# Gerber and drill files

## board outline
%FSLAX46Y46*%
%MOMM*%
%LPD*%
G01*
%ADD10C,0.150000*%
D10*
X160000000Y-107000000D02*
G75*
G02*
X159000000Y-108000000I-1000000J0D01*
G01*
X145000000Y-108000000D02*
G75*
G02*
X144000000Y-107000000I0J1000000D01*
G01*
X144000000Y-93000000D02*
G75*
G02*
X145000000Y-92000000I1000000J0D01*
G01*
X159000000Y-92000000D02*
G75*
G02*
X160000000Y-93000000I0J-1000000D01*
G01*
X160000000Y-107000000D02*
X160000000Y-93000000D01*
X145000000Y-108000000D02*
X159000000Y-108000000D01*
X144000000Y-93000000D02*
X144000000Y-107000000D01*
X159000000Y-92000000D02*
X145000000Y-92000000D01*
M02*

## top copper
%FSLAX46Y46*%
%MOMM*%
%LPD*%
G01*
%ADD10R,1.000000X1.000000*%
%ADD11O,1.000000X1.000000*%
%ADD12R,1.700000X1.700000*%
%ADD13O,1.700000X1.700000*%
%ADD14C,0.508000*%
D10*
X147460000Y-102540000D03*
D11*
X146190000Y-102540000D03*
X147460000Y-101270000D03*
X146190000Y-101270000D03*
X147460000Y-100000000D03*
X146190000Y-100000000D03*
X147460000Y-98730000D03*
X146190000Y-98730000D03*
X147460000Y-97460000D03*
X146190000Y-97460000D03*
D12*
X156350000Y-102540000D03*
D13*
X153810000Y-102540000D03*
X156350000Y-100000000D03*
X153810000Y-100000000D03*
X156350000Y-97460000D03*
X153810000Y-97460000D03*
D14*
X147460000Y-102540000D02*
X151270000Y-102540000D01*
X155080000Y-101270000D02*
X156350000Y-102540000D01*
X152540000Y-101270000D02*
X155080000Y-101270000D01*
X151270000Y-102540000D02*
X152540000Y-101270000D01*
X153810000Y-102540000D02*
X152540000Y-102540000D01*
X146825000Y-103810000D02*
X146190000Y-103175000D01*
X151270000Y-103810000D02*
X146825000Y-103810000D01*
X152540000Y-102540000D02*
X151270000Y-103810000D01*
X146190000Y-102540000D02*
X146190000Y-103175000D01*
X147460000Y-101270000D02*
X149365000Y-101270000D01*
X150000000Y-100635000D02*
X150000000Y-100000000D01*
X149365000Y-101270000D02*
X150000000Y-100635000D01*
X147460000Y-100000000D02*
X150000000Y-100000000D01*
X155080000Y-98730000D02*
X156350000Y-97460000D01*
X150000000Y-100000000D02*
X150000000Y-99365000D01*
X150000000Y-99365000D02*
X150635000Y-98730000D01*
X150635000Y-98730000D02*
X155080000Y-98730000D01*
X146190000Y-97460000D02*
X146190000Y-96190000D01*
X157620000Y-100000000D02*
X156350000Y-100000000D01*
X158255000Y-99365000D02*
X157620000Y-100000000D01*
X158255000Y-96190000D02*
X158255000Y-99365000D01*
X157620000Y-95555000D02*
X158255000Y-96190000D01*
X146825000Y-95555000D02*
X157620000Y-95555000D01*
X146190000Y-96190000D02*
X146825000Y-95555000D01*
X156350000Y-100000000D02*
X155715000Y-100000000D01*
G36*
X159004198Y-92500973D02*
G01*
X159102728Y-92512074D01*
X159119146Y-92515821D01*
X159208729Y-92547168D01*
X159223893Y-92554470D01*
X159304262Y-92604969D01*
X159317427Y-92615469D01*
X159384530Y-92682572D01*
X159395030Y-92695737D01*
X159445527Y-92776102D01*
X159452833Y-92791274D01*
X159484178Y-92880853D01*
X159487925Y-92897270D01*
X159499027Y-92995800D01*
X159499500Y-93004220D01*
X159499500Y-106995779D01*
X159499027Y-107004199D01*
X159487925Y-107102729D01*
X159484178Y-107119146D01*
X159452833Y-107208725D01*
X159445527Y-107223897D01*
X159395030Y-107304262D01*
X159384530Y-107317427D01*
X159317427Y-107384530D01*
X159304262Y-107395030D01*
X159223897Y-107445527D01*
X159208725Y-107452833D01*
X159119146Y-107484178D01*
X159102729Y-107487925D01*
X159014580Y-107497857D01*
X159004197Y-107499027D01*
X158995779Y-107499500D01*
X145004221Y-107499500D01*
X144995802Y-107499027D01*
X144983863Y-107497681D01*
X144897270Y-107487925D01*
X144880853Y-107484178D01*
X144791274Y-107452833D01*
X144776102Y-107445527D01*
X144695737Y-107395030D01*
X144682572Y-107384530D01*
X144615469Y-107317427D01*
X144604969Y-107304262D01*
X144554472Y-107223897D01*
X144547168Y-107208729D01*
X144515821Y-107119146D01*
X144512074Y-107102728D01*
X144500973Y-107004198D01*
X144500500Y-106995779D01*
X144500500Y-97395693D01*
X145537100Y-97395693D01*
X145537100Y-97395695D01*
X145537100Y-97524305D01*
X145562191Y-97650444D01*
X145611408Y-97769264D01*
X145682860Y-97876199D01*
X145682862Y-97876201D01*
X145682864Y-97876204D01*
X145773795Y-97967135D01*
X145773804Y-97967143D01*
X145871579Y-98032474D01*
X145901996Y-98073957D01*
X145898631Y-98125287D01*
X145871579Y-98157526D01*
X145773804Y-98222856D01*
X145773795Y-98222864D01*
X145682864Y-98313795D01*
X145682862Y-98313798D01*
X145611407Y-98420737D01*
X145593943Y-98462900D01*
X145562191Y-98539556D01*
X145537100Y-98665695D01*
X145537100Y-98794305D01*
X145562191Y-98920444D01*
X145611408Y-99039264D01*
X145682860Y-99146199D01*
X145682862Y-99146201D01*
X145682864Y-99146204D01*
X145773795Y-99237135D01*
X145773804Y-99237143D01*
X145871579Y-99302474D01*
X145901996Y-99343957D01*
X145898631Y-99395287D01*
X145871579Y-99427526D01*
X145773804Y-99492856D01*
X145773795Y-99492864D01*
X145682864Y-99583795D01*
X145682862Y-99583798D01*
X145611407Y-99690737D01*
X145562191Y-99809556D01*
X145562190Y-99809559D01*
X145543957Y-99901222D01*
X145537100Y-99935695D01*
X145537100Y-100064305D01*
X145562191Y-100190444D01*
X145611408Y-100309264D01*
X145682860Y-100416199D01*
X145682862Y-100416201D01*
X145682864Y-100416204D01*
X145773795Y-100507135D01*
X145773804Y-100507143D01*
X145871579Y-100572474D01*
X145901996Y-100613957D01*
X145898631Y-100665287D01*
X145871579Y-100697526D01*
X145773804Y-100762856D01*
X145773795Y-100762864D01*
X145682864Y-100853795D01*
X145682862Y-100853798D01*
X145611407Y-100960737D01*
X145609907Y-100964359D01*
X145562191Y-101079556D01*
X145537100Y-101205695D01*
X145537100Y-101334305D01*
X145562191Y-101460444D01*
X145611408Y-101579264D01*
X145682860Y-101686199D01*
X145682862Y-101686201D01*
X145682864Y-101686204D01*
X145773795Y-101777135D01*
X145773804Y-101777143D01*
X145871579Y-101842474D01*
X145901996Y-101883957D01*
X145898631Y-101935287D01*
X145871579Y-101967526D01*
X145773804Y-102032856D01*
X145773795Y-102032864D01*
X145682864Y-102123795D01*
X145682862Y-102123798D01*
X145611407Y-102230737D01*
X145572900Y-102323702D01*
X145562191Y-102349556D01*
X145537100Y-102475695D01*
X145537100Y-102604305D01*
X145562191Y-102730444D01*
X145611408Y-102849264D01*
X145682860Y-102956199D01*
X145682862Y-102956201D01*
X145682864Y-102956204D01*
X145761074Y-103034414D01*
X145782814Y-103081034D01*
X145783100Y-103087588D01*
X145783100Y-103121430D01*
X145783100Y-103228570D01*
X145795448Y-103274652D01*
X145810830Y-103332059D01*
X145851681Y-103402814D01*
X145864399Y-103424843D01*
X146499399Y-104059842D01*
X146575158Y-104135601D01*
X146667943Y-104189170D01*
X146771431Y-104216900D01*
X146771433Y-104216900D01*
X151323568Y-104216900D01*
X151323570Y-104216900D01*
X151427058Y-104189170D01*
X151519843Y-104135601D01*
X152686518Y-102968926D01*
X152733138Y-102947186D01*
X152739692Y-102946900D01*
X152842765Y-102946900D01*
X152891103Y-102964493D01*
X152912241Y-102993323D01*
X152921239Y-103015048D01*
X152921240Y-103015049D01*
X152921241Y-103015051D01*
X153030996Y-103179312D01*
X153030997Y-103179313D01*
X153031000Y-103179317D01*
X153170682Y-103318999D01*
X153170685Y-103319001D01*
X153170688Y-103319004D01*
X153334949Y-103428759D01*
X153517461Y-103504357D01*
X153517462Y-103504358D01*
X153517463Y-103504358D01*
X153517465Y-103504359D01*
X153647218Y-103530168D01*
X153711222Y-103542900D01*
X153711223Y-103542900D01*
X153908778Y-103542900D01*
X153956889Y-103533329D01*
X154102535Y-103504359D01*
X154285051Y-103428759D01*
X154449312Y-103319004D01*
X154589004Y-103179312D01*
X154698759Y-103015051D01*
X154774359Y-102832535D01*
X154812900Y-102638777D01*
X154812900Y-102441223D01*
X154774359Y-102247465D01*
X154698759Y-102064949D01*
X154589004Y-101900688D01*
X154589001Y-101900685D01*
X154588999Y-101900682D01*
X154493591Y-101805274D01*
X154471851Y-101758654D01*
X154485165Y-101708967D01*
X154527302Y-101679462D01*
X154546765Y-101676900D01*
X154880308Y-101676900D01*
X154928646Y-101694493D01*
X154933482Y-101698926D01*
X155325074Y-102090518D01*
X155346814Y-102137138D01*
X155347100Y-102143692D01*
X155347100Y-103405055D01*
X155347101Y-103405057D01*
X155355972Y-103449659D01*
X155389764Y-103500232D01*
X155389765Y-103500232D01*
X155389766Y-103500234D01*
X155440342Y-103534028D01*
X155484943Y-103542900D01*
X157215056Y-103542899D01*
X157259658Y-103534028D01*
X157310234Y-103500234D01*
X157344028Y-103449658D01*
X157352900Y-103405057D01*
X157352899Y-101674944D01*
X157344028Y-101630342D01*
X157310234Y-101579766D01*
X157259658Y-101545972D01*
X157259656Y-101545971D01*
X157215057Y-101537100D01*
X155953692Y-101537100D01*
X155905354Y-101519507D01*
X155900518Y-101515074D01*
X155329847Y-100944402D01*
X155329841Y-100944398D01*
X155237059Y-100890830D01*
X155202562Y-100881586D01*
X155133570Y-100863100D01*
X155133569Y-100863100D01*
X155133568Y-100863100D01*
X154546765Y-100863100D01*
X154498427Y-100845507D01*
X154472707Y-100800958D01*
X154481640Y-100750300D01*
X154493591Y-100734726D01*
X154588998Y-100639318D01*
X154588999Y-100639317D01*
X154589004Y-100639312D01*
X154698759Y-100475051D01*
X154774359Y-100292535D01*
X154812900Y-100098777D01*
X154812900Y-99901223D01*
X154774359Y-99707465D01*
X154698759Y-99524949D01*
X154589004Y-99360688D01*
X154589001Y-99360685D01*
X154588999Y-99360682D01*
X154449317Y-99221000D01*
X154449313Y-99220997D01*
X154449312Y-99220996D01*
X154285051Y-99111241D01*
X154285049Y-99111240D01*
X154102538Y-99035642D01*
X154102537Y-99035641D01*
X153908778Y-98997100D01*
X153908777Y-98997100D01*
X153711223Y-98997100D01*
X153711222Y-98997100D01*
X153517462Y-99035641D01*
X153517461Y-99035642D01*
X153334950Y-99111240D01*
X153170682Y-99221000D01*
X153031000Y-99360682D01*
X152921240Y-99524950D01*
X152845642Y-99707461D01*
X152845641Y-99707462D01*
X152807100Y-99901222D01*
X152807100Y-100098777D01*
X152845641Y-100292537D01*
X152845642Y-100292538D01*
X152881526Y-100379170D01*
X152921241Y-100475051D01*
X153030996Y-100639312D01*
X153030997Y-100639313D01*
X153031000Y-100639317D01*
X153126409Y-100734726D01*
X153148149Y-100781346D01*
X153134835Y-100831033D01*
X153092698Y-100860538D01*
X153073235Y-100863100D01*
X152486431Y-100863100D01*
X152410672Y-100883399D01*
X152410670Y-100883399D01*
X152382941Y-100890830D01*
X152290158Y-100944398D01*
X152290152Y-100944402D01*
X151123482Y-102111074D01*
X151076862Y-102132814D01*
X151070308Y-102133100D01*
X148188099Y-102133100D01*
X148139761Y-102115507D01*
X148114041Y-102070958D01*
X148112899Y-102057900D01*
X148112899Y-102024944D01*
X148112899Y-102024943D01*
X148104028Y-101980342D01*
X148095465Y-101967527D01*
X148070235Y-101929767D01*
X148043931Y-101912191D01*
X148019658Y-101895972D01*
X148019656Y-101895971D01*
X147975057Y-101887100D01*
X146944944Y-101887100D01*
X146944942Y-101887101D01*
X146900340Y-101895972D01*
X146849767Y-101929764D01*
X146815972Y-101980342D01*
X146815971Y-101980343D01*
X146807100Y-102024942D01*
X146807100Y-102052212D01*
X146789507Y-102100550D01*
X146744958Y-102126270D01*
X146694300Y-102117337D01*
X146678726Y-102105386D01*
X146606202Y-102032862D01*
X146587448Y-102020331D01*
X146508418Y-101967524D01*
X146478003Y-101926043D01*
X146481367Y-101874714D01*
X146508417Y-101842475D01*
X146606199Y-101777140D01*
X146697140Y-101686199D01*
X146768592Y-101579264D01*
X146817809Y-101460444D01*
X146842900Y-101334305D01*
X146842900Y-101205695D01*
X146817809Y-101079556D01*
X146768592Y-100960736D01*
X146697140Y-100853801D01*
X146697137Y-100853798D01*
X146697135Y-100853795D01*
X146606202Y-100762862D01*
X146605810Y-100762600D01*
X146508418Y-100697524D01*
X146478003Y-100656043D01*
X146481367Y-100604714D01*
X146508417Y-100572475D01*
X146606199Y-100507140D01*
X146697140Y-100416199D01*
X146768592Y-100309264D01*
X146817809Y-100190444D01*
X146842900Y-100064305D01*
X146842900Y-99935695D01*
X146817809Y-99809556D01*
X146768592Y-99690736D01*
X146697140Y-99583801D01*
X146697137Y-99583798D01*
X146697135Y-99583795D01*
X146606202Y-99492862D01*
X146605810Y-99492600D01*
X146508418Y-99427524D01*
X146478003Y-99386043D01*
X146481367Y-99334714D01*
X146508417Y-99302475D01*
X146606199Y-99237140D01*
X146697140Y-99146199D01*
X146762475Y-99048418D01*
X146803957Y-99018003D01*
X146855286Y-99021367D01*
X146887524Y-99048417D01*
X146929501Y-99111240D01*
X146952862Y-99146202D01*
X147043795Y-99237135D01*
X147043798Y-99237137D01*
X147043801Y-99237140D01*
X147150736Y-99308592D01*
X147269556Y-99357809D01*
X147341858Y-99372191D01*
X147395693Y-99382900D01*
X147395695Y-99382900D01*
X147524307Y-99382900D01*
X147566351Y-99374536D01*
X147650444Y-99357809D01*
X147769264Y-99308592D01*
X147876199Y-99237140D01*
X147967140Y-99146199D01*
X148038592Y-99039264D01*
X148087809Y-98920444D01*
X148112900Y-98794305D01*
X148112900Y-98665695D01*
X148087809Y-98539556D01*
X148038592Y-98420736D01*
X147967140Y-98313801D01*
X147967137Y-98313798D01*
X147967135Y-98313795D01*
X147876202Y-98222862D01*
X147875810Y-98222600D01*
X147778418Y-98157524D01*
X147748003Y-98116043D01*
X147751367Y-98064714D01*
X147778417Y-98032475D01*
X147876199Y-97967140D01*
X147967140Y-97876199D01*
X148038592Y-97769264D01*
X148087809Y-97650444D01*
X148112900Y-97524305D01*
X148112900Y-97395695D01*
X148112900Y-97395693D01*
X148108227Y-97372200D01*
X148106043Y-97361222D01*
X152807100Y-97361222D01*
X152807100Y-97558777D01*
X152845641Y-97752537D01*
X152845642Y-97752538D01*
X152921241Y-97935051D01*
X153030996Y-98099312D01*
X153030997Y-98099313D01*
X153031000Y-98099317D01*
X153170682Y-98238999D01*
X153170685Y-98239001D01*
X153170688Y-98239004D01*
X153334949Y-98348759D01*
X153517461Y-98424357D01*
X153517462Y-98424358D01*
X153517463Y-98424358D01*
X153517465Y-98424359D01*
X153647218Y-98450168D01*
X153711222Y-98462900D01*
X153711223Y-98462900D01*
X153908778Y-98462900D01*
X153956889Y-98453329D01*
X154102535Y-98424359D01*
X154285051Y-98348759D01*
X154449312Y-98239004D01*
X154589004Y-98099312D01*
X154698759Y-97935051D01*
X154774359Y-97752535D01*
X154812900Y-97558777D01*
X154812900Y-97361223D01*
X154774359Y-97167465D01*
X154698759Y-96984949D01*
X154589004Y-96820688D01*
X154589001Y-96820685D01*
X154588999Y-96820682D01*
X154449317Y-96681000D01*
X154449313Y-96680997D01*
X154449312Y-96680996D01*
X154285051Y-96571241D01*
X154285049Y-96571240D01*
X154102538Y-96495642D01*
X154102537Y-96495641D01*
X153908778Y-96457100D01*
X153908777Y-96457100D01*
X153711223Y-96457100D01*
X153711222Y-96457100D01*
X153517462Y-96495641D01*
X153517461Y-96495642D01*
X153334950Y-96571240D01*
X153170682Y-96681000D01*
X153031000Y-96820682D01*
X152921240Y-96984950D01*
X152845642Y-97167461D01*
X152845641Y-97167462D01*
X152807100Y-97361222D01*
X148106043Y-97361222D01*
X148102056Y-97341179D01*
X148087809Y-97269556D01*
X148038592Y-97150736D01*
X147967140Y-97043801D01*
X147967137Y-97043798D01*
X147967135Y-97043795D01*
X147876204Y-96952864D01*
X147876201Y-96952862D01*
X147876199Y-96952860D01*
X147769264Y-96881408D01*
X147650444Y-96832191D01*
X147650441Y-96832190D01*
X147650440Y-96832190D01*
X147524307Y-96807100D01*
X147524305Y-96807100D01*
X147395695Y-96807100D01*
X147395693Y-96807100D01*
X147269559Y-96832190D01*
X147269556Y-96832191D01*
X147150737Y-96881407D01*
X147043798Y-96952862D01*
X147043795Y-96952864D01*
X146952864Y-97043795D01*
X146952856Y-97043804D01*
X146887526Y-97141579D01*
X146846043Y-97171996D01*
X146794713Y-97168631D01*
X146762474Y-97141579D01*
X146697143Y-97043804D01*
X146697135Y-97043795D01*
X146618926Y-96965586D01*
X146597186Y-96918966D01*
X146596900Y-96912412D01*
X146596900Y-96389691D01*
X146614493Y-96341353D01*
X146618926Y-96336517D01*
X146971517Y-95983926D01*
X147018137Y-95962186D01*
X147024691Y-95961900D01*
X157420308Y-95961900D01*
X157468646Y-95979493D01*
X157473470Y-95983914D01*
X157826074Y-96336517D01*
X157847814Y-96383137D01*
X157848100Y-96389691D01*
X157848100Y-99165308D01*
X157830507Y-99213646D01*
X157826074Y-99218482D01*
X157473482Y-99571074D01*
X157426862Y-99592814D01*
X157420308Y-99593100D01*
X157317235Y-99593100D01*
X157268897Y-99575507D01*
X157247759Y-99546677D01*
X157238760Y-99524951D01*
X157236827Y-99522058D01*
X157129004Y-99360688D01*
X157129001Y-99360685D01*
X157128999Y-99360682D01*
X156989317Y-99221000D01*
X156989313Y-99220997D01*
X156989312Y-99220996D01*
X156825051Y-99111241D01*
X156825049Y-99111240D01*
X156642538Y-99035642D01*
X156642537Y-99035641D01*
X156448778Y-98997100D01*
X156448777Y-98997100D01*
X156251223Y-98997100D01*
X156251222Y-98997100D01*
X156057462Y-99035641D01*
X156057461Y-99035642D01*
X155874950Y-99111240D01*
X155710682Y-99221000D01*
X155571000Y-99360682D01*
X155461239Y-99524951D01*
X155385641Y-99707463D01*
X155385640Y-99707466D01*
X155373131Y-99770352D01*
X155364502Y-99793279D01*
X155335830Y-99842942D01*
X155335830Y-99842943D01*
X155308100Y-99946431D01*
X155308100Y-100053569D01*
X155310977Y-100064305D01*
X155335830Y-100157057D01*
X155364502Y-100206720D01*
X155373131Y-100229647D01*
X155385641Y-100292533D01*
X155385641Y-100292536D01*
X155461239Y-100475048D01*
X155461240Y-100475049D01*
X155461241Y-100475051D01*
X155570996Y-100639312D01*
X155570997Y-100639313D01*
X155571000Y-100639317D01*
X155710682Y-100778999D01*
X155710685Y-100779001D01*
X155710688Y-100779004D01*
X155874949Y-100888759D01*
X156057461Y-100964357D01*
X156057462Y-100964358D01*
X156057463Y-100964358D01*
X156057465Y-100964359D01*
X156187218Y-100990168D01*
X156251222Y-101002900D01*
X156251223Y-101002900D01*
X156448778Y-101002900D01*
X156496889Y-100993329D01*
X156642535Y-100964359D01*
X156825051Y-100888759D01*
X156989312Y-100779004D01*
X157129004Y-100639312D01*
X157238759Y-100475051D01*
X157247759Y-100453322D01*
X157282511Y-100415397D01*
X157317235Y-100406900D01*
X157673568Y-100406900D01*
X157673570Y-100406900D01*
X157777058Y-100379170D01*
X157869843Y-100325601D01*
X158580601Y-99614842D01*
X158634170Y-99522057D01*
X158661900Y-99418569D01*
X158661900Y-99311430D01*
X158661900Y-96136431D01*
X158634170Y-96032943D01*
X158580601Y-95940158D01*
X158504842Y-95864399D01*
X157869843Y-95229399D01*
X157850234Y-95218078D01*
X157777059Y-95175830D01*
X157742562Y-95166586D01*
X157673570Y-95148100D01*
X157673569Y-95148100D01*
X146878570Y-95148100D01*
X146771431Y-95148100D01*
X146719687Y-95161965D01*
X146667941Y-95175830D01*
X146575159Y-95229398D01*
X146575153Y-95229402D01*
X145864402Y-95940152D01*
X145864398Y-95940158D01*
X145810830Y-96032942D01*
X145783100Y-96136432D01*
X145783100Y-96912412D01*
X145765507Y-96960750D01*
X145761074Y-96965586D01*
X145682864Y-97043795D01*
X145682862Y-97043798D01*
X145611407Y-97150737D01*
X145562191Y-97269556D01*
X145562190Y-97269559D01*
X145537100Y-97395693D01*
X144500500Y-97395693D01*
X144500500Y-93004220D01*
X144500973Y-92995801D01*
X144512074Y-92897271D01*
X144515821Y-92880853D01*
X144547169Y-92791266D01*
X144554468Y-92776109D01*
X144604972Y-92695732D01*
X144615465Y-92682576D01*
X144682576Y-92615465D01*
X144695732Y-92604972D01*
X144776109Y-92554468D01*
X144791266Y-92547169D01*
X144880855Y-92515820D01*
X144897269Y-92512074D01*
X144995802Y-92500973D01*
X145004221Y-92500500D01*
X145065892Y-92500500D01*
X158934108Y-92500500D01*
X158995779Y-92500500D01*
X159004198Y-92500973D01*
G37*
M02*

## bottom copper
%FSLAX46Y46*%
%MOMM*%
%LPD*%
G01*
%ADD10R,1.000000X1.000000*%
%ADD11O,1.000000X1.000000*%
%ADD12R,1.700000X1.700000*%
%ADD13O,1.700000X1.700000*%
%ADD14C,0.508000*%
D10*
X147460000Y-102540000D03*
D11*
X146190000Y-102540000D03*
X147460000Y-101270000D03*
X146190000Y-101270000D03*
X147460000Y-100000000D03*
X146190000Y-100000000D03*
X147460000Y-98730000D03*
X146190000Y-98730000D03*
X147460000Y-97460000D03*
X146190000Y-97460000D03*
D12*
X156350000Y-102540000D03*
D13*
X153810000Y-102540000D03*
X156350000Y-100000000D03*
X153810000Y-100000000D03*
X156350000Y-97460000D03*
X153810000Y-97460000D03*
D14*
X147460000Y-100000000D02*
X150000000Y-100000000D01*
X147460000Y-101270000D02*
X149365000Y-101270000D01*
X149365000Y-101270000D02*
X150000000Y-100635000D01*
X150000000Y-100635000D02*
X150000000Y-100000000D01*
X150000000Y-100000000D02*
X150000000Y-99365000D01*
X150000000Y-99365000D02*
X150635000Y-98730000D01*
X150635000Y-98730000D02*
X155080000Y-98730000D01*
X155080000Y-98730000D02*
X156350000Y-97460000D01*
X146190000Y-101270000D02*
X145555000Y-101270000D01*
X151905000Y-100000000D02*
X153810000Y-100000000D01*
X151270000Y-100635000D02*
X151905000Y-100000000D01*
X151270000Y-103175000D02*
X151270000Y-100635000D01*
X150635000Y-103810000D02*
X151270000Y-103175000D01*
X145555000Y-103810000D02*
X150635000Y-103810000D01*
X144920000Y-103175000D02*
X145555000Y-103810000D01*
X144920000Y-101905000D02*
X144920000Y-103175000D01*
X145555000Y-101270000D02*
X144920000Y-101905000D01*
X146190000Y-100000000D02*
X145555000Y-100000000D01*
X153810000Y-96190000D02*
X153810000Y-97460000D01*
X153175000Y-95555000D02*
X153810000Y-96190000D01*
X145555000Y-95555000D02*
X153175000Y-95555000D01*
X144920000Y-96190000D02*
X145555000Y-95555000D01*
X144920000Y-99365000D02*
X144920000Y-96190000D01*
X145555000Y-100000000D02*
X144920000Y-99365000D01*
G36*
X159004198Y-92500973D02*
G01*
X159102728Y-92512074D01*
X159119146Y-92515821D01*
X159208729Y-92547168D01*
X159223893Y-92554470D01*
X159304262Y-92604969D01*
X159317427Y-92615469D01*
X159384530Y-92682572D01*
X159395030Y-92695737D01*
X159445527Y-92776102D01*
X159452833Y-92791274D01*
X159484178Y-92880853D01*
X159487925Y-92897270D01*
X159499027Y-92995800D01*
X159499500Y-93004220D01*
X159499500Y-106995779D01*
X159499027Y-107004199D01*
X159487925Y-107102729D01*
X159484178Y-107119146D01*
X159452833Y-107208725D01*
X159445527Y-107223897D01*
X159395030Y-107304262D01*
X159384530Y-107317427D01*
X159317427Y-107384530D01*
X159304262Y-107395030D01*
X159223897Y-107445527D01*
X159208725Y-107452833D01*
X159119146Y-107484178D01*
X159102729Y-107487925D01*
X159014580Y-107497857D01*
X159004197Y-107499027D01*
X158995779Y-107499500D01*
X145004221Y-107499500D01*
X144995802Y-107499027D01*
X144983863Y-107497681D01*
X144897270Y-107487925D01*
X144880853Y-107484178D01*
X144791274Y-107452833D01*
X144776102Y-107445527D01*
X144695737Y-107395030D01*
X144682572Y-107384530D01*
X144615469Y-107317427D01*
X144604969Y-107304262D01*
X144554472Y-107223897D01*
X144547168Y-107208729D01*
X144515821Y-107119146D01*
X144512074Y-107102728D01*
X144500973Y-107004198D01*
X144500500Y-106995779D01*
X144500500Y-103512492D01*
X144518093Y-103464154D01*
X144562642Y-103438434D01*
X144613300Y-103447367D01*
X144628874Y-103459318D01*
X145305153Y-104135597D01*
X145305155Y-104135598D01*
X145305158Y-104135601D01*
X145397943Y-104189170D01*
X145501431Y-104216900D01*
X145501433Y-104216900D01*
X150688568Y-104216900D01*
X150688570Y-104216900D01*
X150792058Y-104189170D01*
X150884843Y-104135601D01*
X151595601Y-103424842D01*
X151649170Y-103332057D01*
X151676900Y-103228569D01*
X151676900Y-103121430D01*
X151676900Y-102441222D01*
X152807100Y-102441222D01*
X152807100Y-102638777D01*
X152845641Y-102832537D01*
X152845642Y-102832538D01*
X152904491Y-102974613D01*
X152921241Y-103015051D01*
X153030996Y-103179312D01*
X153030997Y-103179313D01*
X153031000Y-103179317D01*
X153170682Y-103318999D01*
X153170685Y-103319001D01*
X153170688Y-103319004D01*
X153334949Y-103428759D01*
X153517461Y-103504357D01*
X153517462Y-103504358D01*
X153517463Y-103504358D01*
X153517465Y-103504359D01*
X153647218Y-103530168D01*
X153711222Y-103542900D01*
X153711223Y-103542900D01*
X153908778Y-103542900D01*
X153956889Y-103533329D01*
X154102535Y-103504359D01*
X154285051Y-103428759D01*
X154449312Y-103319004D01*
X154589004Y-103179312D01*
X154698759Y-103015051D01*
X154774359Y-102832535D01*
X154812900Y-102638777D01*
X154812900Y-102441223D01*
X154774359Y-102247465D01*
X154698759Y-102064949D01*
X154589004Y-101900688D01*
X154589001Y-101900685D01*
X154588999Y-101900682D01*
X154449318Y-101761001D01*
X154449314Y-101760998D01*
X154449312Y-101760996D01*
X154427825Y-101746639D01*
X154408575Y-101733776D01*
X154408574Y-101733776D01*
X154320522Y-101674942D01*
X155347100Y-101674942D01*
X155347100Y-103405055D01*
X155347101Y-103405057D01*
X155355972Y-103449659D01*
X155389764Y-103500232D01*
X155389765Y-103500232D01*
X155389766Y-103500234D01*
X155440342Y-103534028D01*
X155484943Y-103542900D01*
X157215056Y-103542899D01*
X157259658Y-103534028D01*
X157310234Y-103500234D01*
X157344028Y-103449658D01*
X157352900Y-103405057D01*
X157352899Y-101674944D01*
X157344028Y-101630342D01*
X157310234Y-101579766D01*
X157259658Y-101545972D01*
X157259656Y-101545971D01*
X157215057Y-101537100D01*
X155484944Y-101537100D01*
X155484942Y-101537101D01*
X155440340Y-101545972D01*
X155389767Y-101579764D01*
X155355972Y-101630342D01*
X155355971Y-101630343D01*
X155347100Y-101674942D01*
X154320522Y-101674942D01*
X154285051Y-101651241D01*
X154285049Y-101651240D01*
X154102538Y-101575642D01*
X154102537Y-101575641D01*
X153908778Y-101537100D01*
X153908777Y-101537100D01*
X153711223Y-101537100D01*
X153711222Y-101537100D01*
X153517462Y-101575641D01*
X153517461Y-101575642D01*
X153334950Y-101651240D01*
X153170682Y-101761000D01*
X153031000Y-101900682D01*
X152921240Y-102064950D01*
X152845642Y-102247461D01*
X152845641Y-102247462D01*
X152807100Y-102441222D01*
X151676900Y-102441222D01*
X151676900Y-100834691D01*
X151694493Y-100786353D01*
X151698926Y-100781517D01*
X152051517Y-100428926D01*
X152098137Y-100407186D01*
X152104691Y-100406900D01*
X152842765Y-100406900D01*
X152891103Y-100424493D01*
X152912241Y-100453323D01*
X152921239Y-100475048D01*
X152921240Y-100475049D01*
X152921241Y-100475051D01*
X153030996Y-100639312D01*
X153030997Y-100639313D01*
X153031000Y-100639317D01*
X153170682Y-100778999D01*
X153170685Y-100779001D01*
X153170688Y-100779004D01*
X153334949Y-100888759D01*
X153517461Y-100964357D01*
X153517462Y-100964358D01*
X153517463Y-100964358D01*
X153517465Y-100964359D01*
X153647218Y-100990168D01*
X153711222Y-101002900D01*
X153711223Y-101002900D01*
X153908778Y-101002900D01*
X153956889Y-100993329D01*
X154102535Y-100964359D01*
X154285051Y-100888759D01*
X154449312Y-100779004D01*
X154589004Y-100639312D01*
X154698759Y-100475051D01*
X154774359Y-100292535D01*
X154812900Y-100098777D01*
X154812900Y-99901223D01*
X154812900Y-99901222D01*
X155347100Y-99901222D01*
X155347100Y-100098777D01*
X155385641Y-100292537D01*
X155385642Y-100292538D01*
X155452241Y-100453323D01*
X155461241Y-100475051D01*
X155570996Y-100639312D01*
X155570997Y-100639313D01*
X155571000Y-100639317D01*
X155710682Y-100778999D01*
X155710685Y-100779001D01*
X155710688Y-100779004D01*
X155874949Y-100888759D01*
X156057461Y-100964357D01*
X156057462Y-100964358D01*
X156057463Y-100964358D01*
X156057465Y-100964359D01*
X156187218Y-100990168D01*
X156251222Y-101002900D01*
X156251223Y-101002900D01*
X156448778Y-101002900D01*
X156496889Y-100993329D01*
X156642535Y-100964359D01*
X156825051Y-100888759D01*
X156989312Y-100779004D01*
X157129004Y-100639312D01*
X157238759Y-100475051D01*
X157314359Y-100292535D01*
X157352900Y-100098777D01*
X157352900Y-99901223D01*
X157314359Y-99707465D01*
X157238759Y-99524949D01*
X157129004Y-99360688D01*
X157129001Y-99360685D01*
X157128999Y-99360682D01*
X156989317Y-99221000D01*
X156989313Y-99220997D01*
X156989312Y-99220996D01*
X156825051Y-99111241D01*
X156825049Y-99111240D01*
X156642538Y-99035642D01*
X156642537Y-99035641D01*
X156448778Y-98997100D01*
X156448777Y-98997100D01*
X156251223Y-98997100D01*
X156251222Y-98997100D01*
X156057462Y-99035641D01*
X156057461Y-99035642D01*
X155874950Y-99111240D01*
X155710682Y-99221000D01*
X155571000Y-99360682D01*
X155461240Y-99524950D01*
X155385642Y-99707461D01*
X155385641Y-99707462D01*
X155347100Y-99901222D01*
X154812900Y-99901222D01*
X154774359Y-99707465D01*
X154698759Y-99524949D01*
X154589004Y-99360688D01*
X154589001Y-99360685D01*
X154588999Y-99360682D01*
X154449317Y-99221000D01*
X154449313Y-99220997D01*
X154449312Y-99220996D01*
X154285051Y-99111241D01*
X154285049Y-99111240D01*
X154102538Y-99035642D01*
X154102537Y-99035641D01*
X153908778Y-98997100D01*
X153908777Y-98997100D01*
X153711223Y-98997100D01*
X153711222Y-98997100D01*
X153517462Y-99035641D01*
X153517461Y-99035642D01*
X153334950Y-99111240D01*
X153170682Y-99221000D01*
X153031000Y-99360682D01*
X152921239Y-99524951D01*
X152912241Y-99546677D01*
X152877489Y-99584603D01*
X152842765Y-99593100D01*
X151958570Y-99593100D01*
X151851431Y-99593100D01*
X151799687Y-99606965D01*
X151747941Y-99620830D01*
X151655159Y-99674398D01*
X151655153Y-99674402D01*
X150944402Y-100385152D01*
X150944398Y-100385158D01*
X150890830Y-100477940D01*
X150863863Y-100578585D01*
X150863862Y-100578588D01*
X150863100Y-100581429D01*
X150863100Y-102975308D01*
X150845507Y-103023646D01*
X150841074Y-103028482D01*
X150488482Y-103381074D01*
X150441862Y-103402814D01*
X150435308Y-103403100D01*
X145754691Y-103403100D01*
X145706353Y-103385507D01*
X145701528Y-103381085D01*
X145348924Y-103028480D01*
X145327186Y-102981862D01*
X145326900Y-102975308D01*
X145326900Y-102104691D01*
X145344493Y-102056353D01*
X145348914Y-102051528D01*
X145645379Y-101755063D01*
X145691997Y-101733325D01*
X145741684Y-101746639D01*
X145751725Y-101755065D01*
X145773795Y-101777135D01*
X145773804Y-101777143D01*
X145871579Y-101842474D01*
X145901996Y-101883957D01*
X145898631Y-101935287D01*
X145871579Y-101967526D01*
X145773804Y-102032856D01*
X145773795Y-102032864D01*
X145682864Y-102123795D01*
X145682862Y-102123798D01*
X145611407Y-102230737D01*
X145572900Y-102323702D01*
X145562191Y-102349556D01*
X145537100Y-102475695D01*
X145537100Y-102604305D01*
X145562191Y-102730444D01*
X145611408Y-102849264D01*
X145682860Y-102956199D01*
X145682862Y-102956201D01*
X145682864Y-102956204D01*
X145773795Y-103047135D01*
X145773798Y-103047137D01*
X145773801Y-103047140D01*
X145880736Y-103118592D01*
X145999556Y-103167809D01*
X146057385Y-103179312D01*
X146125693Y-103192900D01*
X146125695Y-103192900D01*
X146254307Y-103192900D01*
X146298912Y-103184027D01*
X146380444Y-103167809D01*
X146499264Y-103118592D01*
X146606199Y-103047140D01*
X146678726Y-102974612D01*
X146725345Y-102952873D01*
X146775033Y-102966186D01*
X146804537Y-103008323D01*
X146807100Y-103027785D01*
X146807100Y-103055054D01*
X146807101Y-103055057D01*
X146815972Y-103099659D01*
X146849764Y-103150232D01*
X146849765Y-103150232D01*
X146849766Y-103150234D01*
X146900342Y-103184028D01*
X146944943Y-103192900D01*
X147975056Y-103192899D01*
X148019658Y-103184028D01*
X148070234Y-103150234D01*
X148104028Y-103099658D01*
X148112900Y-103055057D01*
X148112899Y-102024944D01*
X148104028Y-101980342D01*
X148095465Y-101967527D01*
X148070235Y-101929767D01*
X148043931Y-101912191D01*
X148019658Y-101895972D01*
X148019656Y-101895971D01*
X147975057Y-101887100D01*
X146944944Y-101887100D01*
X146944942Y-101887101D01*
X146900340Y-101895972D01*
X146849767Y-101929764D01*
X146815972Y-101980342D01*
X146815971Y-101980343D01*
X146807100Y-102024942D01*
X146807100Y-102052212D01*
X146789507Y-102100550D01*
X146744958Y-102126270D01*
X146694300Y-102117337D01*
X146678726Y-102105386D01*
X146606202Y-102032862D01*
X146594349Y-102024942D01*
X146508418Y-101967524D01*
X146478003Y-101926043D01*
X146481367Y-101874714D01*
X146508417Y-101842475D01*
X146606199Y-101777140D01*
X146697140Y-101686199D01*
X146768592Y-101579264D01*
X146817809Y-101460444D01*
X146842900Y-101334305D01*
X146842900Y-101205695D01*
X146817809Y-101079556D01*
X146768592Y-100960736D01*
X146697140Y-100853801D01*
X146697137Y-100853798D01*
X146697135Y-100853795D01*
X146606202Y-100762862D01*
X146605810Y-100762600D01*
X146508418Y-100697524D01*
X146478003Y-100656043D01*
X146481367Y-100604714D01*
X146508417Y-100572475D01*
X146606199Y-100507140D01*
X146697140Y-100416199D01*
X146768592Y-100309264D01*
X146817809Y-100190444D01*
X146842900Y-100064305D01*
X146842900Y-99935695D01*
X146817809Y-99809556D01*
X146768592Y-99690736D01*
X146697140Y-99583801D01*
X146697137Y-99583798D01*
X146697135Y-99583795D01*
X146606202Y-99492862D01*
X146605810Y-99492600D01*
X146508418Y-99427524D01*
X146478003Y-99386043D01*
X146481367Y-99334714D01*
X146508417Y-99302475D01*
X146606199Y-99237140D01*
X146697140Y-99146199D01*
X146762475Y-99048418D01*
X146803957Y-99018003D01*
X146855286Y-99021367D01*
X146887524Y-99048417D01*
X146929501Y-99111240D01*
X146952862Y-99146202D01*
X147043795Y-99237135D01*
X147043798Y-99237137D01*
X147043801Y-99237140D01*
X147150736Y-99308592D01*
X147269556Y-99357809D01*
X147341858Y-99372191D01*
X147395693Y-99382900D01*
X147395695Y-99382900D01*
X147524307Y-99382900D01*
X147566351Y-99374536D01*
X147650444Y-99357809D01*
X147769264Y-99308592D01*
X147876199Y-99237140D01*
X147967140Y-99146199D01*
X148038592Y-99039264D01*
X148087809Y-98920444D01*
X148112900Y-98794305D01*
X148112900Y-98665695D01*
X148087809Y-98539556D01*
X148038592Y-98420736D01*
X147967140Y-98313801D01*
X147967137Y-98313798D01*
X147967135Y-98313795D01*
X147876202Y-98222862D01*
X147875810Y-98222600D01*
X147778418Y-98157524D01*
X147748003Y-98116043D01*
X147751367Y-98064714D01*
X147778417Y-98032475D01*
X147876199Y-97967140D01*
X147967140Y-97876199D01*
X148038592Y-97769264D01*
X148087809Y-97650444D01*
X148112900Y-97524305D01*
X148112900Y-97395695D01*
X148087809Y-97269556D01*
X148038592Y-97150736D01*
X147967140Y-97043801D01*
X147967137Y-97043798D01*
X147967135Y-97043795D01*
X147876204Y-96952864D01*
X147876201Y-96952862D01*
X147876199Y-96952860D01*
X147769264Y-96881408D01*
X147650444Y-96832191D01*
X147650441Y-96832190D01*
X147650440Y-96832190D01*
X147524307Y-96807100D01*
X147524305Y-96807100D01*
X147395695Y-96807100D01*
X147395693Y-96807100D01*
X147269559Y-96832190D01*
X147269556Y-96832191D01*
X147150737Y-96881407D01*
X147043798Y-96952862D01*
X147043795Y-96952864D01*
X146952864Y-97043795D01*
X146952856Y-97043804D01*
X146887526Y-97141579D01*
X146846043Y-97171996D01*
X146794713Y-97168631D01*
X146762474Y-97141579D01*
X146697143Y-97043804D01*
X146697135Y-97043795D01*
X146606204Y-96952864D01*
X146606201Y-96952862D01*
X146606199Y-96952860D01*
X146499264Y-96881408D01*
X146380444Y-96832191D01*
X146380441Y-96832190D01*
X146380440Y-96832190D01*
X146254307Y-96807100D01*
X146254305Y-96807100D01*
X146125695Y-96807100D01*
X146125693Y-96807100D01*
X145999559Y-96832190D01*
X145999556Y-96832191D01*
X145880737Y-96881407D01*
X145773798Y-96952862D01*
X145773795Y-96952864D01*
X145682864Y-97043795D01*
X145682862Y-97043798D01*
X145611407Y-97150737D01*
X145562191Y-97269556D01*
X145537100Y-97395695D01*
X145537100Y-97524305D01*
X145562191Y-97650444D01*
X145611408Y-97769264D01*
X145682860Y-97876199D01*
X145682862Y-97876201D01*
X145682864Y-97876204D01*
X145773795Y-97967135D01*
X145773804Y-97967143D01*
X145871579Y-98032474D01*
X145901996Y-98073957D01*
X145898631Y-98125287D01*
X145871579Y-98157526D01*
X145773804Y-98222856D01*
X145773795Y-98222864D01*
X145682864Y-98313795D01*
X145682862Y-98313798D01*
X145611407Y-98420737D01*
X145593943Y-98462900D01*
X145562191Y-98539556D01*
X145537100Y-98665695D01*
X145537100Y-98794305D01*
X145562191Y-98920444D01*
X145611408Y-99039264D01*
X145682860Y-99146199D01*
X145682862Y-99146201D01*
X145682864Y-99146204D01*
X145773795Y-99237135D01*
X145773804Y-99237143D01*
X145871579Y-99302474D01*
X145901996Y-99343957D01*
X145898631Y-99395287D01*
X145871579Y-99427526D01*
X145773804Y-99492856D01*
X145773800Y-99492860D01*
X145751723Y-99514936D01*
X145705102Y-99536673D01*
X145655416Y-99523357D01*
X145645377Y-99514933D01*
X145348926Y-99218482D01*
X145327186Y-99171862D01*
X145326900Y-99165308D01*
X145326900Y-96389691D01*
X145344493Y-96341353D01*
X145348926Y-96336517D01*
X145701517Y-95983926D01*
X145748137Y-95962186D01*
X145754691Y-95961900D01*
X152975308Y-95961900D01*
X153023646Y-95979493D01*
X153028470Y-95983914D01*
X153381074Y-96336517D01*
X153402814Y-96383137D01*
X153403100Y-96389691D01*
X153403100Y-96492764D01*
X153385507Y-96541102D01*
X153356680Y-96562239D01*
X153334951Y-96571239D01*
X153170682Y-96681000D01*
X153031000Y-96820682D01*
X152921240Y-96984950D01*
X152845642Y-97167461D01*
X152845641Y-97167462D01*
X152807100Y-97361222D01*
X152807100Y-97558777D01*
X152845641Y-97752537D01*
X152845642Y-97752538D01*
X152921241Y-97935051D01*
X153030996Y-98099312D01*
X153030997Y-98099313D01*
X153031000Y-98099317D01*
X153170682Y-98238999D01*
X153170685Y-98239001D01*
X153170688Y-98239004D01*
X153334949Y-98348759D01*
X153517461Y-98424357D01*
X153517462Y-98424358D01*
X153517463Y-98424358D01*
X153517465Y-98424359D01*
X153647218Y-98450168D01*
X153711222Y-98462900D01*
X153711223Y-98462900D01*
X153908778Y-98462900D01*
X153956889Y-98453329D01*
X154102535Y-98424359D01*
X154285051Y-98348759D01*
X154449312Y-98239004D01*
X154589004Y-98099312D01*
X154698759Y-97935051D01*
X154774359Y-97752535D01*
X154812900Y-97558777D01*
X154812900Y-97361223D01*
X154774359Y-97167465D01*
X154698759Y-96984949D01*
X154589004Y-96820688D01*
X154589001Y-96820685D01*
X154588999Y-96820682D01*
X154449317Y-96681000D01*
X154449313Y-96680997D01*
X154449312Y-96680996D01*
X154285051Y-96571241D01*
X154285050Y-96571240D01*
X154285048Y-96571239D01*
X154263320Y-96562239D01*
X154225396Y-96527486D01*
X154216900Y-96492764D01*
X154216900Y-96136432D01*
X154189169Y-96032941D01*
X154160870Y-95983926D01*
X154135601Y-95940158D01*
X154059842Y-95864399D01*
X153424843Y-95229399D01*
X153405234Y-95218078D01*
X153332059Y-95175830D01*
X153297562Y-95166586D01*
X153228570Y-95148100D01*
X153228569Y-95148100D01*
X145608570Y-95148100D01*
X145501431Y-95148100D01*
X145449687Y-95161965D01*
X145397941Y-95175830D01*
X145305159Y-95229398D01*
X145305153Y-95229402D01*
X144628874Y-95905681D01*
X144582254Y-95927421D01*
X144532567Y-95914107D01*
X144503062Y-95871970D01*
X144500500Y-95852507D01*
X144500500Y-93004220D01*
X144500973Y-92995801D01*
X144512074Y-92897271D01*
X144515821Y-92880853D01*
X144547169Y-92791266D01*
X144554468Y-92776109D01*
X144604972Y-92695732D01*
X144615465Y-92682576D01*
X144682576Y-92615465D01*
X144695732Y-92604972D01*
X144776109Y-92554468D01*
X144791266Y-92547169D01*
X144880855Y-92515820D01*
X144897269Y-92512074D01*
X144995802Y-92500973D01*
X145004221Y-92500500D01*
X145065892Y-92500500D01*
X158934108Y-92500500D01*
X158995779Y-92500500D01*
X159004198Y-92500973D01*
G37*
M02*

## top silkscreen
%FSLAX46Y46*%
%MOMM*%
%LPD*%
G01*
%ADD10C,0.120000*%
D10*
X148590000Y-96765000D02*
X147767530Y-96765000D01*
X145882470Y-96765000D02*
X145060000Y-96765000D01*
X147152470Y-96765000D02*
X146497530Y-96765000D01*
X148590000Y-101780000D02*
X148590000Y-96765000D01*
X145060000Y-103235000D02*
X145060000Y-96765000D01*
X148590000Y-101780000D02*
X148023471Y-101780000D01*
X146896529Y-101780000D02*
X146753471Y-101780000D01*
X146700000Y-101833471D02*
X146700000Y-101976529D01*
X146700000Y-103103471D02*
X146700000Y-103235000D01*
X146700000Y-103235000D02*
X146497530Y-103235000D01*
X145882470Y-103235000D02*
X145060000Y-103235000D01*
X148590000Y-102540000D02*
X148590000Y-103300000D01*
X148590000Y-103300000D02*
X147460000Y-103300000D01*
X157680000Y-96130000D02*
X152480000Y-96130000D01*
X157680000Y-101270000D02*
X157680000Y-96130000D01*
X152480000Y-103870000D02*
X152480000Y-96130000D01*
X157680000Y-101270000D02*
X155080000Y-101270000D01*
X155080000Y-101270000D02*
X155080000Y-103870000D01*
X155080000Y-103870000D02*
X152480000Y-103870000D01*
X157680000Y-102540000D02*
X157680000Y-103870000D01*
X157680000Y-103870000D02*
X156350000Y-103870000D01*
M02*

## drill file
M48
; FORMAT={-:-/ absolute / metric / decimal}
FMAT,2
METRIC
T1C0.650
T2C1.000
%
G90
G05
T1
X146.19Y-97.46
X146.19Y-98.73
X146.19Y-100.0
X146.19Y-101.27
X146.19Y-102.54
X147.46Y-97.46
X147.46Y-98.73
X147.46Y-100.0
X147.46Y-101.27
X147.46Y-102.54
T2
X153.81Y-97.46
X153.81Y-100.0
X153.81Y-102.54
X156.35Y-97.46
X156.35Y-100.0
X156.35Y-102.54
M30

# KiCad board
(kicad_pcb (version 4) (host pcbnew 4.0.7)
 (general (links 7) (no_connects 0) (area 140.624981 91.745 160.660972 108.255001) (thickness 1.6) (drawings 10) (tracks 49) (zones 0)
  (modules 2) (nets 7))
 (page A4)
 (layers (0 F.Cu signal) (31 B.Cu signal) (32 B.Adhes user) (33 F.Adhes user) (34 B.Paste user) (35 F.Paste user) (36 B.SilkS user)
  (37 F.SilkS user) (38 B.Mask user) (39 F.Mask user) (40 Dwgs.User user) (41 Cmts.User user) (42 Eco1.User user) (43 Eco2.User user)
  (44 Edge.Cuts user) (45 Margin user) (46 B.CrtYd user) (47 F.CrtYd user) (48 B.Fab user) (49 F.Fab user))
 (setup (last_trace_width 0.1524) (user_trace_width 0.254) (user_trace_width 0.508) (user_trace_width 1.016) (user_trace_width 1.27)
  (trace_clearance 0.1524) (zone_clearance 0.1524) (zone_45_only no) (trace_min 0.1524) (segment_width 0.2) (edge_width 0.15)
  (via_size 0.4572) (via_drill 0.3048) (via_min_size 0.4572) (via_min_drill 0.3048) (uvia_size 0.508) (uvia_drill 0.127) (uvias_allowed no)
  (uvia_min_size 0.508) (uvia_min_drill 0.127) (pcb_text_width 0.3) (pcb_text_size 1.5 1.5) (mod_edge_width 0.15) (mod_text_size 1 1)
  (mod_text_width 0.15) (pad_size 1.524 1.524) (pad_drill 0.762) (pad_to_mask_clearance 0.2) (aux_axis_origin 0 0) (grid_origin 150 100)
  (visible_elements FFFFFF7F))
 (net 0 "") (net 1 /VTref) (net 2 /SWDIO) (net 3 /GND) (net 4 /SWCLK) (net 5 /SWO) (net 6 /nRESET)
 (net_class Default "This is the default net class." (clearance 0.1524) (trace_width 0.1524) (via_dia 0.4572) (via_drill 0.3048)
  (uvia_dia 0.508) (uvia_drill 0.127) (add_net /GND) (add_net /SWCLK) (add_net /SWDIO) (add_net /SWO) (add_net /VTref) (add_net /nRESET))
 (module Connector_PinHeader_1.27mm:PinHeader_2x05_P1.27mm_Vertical (layer F.Cu) (at 147.46 102.54 180)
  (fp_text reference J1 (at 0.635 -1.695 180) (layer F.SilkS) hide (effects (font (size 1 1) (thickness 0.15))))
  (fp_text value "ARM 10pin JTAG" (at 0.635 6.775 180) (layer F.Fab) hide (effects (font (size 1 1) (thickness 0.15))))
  (fp_line (start -1.13 5.775) (end -0.30753 5.775) (layer F.SilkS) (width 0.12))
  (fp_line (start 1.57753 5.775) (end 2.4 5.775) (layer F.SilkS) (width 0.12))
  (fp_line (start 0.30753 5.775) (end 0.96247 5.775) (layer F.SilkS) (width 0.12))
  (fp_line (start -1.13 0.76) (end -1.13 5.775) (layer F.SilkS) (width 0.12))
  (fp_line (start 2.4 -0.695) (end 2.4 5.775) (layer F.SilkS) (width 0.12))
  (fp_line (start -1.13 0.76) (end -0.563471 0.76) (layer F.SilkS) (width 0.12))
  (fp_line (start 0.563471 0.76) (end 0.706529 0.76) (layer F.SilkS) (width 0.12))
  (fp_line (start 0.76 0.706529) (end 0.76 0.563471) (layer F.SilkS) (width 0.12))
  (fp_line (start 0.76 -0.563471) (end 0.76 -0.695) (layer F.SilkS) (width 0.12))
  (fp_line (start 0.76 -0.695) (end 0.96247 -0.695) (layer F.SilkS) (width 0.12))
  (fp_line (start 1.57753 -0.695) (end 2.4 -0.695) (layer F.SilkS) (width 0.12))
  (fp_line (start -1.13 0) (end -1.13 -0.76) (layer F.SilkS) (width 0.12))
  (fp_line (start -1.13 -0.76) (end 0 -0.76) (layer F.SilkS) (width 0.12))
  (pad 1 thru_hole rect (at 0 0 180) (size 1 1) (drill 0.65) (layers *.Cu *.Mask) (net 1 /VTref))
  (pad 2 thru_hole oval (at 1.27 0 180) (size 1 1) (drill 0.65) (layers *.Cu *.Mask) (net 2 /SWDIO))
  (pad 3 thru_hole oval (at 0 1.27 180) (size 1 1) (drill 0.65) (layers *.Cu *.Mask) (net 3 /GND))
  (pad 4 thru_hole oval (at 1.27 1.27 180) (size 1 1) (drill 0.65) (layers *.Cu *.Mask) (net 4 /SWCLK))
  (pad 5 thru_hole oval (at 0 2.54 180) (size 1 1) (drill 0.65) (layers *.Cu *.Mask) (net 3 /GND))
  (pad 6 thru_hole oval (at 1.27 2.54 180) (size 1 1) (drill 0.65) (layers *.Cu *.Mask) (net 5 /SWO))
  (pad 7 thru_hole oval (at 0 3.81 180) (size 1 1) (drill 0.65) (layers *.Cu *.Mask))
  (pad 8 thru_hole oval (at 1.27 3.81 180) (size 1 1) (drill 0.65) (layers *.Cu *.Mask))
  (pad 9 thru_hole oval (at 0 5.08 180) (size 1 1) (drill 0.65) (layers *.Cu *.Mask))
  (pad 10 thru_hole oval (at 1.27 5.08 180) (size 1 1) (drill 0.65) (layers *.Cu *.Mask) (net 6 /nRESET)))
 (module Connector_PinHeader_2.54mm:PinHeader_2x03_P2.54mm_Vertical (layer F.Cu) (at 156.35 102.54 180)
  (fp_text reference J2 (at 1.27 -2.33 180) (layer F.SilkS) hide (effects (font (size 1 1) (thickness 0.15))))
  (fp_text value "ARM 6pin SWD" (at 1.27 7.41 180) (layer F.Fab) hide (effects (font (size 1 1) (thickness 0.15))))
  (fp_line (start -1.33 6.41) (end 3.87 6.41) (layer F.SilkS) (width 0.12))
  (fp_line (start -1.33 1.27) (end -1.33 6.41) (layer F.SilkS) (width 0.12))
  (fp_line (start 3.87 -1.33) (end 3.87 6.41) (layer F.SilkS) (width 0.12))
  (fp_line (start -1.33 1.27) (end 1.27 1.27) (layer F.SilkS) (width 0.12))
  (fp_line (start 1.27 1.27) (end 1.27 -1.33) (layer F.SilkS) (width 0.12))
  (fp_line (start 1.27 -1.33) (end 3.87 -1.33) (layer F.SilkS) (width 0.12))
  (fp_line (start -1.33 0) (end -1.33 -1.33) (layer F.SilkS) (width 0.12))
  (fp_line (start -1.33 -1.33) (end 0 -1.33) (layer F.SilkS) (width 0.12))
  (pad 1 thru_hole rect (at 0 0 180) (size 1.7 1.7) (drill 1) (layers *.Cu *.Mask) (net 1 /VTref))
  (pad 2 thru_hole oval (at 2.54 0 180) (size 1.7 1.7) (drill 1) (layers *.Cu *.Mask) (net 2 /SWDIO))
  (pad 3 thru_hole oval (at 0 2.54 180) (size 1.7 1.7) (drill 1) (layers *.Cu *.Mask) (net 6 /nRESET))
  (pad 4 thru_hole oval (at 2.54 2.54 180) (size 1.7 1.7) (drill 1) (layers *.Cu *.Mask) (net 4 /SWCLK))
  (pad 5 thru_hole oval (at 0 5.08 180) (size 1.7 1.7) (drill 1) (layers *.Cu *.Mask) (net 3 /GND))
  (pad 6 thru_hole oval (at 2.54 5.08 180) (size 1.7 1.7) (drill 1) (layers *.Cu *.Mask) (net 5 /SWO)))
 (gr_arc (start 159 107) (end 160 107) (angle 90) (layer Edge.Cuts) (width 0.15))
 (gr_arc (start 145 107) (end 145 108) (angle 90) (layer Edge.Cuts) (width 0.15))
 (gr_arc (start 145 93) (end 144 93) (angle 90) (layer Edge.Cuts) (width 0.15))
 (gr_arc (start 159 93) (end 159 92) (angle 90) (layer Edge.Cuts) (width 0.15))
 (gr_line (start 160 107) (end 160 93) (angle 90) (layer Edge.Cuts) (width 0.15))
 (gr_line (start 145 108) (end 159 108) (angle 90) (layer Edge.Cuts) (width 0.15))
 (gr_line (start 144 93) (end 144 107) (angle 90) (layer Edge.Cuts) (width 0.15))
 (gr_line (start 159 92) (end 145 92) (angle 90) (layer Edge.Cuts) (width 0.15))
 (segment (start 147.46 102.54) (end 151.27 102.54) (width 0.508) (layer F.Cu) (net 1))
 (segment (start 155.08 101.27) (end 156.35 102.54) (width 0.508) (layer F.Cu) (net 1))
 (segment (start 152.54 101.27) (end 155.08 101.27) (width 0.508) (layer F.Cu) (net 1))
 (segment (start 151.27 102.54) (end 152.54 101.27) (width 0.508) (layer F.Cu) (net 1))
 (segment (start 153.81 102.54) (end 152.54 102.54) (width 0.508) (layer F.Cu) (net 2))
 (segment (start 146.825 103.81) (end 146.19 103.175) (width 0.508) (layer F.Cu) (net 2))
 (segment (start 151.27 103.81) (end 146.825 103.81) (width 0.508) (layer F.Cu) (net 2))
 (segment (start 152.54 102.54) (end 151.27 103.81) (width 0.508) (layer F.Cu) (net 2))
 (segment (start 146.19 102.54) (end 146.19 103.175) (width 0.508) (layer F.Cu) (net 2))
 (segment (start 147.46 101.27) (end 149.365 101.27) (width 0.508) (layer F.Cu) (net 3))
 (segment (start 150 100.635) (end 150 100) (width 0.508) (layer F.Cu) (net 3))
 (segment (start 149.365 101.27) (end 150 100.635) (width 0.508) (layer F.Cu) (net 3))
 (segment (start 147.46 100) (end 150 100) (width 0.508) (layer F.Cu) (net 3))
 (segment (start 155.08 98.73) (end 156.35 97.46) (width 0.508) (layer F.Cu) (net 3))
 (segment (start 150 100) (end 150 99.365) (width 0.508) (layer F.Cu) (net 3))
 (segment (start 150 99.365) (end 150.635 98.73) (width 0.508) (layer F.Cu) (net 3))
 (segment (start 150.635 98.73) (end 155.08 98.73) (width 0.508) (layer F.Cu) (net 3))
 (segment (start 147.46 100) (end 150 100) (width 0.508) (layer B.Cu) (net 3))
 (segment (start 147.46 101.27) (end 149.365 101.27) (width 0.508) (layer B.Cu) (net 3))
 (segment (start 149.365 101.27) (end 150 100.635) (width 0.508) (layer B.Cu) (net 3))
 (segment (start 150 100.635) (end 150 100) (width 0.508) (layer B.Cu) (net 3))
 (segment (start 150 100) (end 150 99.365) (width 0.508) (layer B.Cu) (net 3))
 (segment (start 150 99.365) (end 150.635 98.73) (width 0.508) (layer B.Cu) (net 3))
 (segment (start 150.635 98.73) (end 155.08 98.73) (width 0.508) (layer B.Cu) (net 3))
 (segment (start 155.08 98.73) (end 156.35 97.46) (width 0.508) (layer B.Cu) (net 3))
 (segment (start 146.19 101.27) (end 145.555 101.27) (width 0.508) (layer B.Cu) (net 4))
 (segment (start 151.905 100) (end 153.81 100) (width 0.508) (layer B.Cu) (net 4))
 (segment (start 151.27 100.635) (end 151.905 100) (width 0.508) (layer B.Cu) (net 4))
 (segment (start 151.27 103.175) (end 151.27 100.635) (width 0.508) (layer B.Cu) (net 4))
 (segment (start 150.635 103.81) (end 151.27 103.175) (width 0.508) (layer B.Cu) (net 4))
 (segment (start 145.555 103.81) (end 150.635 103.81) (width 0.508) (layer B.Cu) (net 4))
 (segment (start 144.92 103.175) (end 145.555 103.81) (width 0.508) (layer B.Cu) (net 4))
 (segment (start 144.92 101.905) (end 144.92 103.175) (width 0.508) (layer B.Cu) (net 4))
 (segment (start 145.555 101.27) (end 144.92 101.905) (width 0.508) (layer B.Cu) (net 4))
 (segment (start 146.19 100) (end 145.555 100) (width 0.508) (layer B.Cu) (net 5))
 (segment (start 153.81 96.19) (end 153.81 97.46) (width 0.508) (layer B.Cu) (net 5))
 (segment (start 153.175 95.555) (end 153.81 96.19) (width 0.508) (layer B.Cu) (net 5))
 (segment (start 145.555 95.555) (end 153.175 95.555) (width 0.508) (layer B.Cu) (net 5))
 (segment (start 144.92 96.19) (end 145.555 95.555) (width 0.508) (layer B.Cu) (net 5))
 (segment (start 144.92 99.365) (end 144.92 96.19) (width 0.508) (layer B.Cu) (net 5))
 (segment (start 145.555 100) (end 144.92 99.365) (width 0.508) (layer B.Cu) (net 5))
 (segment (start 146.19 97.46) (end 146.19 96.19) (width 0.508) (layer F.Cu) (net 6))
 (segment (start 157.62 100) (end 156.35 100) (width 0.508) (layer F.Cu) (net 6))
 (segment (start 158.255 99.365) (end 157.62 100) (width 0.508) (layer F.Cu) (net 6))
 (segment (start 158.255 96.19) (end 158.255 99.365) (width 0.508) (layer F.Cu) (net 6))
 (segment (start 157.62 95.555) (end 158.255 96.19) (width 0.508) (layer F.Cu) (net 6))
 (segment (start 146.825 95.555) (end 157.62 95.555) (width 0.508) (layer F.Cu) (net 6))
 (segment (start 146.19 96.19) (end 146.825 95.555) (width 0.508) (layer F.Cu) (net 6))
 (segment (start 156.35 100) (end 155.715 100) (width 0.508) (layer F.Cu) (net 6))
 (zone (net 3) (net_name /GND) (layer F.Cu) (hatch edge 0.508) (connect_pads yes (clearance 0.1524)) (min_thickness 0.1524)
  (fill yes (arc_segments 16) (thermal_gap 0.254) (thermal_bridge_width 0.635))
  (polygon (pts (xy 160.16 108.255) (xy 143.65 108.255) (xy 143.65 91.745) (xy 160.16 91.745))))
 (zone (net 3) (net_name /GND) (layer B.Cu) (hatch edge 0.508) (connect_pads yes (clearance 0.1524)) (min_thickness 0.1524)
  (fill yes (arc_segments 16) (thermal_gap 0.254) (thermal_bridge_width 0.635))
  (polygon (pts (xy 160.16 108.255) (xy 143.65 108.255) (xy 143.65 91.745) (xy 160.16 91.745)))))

